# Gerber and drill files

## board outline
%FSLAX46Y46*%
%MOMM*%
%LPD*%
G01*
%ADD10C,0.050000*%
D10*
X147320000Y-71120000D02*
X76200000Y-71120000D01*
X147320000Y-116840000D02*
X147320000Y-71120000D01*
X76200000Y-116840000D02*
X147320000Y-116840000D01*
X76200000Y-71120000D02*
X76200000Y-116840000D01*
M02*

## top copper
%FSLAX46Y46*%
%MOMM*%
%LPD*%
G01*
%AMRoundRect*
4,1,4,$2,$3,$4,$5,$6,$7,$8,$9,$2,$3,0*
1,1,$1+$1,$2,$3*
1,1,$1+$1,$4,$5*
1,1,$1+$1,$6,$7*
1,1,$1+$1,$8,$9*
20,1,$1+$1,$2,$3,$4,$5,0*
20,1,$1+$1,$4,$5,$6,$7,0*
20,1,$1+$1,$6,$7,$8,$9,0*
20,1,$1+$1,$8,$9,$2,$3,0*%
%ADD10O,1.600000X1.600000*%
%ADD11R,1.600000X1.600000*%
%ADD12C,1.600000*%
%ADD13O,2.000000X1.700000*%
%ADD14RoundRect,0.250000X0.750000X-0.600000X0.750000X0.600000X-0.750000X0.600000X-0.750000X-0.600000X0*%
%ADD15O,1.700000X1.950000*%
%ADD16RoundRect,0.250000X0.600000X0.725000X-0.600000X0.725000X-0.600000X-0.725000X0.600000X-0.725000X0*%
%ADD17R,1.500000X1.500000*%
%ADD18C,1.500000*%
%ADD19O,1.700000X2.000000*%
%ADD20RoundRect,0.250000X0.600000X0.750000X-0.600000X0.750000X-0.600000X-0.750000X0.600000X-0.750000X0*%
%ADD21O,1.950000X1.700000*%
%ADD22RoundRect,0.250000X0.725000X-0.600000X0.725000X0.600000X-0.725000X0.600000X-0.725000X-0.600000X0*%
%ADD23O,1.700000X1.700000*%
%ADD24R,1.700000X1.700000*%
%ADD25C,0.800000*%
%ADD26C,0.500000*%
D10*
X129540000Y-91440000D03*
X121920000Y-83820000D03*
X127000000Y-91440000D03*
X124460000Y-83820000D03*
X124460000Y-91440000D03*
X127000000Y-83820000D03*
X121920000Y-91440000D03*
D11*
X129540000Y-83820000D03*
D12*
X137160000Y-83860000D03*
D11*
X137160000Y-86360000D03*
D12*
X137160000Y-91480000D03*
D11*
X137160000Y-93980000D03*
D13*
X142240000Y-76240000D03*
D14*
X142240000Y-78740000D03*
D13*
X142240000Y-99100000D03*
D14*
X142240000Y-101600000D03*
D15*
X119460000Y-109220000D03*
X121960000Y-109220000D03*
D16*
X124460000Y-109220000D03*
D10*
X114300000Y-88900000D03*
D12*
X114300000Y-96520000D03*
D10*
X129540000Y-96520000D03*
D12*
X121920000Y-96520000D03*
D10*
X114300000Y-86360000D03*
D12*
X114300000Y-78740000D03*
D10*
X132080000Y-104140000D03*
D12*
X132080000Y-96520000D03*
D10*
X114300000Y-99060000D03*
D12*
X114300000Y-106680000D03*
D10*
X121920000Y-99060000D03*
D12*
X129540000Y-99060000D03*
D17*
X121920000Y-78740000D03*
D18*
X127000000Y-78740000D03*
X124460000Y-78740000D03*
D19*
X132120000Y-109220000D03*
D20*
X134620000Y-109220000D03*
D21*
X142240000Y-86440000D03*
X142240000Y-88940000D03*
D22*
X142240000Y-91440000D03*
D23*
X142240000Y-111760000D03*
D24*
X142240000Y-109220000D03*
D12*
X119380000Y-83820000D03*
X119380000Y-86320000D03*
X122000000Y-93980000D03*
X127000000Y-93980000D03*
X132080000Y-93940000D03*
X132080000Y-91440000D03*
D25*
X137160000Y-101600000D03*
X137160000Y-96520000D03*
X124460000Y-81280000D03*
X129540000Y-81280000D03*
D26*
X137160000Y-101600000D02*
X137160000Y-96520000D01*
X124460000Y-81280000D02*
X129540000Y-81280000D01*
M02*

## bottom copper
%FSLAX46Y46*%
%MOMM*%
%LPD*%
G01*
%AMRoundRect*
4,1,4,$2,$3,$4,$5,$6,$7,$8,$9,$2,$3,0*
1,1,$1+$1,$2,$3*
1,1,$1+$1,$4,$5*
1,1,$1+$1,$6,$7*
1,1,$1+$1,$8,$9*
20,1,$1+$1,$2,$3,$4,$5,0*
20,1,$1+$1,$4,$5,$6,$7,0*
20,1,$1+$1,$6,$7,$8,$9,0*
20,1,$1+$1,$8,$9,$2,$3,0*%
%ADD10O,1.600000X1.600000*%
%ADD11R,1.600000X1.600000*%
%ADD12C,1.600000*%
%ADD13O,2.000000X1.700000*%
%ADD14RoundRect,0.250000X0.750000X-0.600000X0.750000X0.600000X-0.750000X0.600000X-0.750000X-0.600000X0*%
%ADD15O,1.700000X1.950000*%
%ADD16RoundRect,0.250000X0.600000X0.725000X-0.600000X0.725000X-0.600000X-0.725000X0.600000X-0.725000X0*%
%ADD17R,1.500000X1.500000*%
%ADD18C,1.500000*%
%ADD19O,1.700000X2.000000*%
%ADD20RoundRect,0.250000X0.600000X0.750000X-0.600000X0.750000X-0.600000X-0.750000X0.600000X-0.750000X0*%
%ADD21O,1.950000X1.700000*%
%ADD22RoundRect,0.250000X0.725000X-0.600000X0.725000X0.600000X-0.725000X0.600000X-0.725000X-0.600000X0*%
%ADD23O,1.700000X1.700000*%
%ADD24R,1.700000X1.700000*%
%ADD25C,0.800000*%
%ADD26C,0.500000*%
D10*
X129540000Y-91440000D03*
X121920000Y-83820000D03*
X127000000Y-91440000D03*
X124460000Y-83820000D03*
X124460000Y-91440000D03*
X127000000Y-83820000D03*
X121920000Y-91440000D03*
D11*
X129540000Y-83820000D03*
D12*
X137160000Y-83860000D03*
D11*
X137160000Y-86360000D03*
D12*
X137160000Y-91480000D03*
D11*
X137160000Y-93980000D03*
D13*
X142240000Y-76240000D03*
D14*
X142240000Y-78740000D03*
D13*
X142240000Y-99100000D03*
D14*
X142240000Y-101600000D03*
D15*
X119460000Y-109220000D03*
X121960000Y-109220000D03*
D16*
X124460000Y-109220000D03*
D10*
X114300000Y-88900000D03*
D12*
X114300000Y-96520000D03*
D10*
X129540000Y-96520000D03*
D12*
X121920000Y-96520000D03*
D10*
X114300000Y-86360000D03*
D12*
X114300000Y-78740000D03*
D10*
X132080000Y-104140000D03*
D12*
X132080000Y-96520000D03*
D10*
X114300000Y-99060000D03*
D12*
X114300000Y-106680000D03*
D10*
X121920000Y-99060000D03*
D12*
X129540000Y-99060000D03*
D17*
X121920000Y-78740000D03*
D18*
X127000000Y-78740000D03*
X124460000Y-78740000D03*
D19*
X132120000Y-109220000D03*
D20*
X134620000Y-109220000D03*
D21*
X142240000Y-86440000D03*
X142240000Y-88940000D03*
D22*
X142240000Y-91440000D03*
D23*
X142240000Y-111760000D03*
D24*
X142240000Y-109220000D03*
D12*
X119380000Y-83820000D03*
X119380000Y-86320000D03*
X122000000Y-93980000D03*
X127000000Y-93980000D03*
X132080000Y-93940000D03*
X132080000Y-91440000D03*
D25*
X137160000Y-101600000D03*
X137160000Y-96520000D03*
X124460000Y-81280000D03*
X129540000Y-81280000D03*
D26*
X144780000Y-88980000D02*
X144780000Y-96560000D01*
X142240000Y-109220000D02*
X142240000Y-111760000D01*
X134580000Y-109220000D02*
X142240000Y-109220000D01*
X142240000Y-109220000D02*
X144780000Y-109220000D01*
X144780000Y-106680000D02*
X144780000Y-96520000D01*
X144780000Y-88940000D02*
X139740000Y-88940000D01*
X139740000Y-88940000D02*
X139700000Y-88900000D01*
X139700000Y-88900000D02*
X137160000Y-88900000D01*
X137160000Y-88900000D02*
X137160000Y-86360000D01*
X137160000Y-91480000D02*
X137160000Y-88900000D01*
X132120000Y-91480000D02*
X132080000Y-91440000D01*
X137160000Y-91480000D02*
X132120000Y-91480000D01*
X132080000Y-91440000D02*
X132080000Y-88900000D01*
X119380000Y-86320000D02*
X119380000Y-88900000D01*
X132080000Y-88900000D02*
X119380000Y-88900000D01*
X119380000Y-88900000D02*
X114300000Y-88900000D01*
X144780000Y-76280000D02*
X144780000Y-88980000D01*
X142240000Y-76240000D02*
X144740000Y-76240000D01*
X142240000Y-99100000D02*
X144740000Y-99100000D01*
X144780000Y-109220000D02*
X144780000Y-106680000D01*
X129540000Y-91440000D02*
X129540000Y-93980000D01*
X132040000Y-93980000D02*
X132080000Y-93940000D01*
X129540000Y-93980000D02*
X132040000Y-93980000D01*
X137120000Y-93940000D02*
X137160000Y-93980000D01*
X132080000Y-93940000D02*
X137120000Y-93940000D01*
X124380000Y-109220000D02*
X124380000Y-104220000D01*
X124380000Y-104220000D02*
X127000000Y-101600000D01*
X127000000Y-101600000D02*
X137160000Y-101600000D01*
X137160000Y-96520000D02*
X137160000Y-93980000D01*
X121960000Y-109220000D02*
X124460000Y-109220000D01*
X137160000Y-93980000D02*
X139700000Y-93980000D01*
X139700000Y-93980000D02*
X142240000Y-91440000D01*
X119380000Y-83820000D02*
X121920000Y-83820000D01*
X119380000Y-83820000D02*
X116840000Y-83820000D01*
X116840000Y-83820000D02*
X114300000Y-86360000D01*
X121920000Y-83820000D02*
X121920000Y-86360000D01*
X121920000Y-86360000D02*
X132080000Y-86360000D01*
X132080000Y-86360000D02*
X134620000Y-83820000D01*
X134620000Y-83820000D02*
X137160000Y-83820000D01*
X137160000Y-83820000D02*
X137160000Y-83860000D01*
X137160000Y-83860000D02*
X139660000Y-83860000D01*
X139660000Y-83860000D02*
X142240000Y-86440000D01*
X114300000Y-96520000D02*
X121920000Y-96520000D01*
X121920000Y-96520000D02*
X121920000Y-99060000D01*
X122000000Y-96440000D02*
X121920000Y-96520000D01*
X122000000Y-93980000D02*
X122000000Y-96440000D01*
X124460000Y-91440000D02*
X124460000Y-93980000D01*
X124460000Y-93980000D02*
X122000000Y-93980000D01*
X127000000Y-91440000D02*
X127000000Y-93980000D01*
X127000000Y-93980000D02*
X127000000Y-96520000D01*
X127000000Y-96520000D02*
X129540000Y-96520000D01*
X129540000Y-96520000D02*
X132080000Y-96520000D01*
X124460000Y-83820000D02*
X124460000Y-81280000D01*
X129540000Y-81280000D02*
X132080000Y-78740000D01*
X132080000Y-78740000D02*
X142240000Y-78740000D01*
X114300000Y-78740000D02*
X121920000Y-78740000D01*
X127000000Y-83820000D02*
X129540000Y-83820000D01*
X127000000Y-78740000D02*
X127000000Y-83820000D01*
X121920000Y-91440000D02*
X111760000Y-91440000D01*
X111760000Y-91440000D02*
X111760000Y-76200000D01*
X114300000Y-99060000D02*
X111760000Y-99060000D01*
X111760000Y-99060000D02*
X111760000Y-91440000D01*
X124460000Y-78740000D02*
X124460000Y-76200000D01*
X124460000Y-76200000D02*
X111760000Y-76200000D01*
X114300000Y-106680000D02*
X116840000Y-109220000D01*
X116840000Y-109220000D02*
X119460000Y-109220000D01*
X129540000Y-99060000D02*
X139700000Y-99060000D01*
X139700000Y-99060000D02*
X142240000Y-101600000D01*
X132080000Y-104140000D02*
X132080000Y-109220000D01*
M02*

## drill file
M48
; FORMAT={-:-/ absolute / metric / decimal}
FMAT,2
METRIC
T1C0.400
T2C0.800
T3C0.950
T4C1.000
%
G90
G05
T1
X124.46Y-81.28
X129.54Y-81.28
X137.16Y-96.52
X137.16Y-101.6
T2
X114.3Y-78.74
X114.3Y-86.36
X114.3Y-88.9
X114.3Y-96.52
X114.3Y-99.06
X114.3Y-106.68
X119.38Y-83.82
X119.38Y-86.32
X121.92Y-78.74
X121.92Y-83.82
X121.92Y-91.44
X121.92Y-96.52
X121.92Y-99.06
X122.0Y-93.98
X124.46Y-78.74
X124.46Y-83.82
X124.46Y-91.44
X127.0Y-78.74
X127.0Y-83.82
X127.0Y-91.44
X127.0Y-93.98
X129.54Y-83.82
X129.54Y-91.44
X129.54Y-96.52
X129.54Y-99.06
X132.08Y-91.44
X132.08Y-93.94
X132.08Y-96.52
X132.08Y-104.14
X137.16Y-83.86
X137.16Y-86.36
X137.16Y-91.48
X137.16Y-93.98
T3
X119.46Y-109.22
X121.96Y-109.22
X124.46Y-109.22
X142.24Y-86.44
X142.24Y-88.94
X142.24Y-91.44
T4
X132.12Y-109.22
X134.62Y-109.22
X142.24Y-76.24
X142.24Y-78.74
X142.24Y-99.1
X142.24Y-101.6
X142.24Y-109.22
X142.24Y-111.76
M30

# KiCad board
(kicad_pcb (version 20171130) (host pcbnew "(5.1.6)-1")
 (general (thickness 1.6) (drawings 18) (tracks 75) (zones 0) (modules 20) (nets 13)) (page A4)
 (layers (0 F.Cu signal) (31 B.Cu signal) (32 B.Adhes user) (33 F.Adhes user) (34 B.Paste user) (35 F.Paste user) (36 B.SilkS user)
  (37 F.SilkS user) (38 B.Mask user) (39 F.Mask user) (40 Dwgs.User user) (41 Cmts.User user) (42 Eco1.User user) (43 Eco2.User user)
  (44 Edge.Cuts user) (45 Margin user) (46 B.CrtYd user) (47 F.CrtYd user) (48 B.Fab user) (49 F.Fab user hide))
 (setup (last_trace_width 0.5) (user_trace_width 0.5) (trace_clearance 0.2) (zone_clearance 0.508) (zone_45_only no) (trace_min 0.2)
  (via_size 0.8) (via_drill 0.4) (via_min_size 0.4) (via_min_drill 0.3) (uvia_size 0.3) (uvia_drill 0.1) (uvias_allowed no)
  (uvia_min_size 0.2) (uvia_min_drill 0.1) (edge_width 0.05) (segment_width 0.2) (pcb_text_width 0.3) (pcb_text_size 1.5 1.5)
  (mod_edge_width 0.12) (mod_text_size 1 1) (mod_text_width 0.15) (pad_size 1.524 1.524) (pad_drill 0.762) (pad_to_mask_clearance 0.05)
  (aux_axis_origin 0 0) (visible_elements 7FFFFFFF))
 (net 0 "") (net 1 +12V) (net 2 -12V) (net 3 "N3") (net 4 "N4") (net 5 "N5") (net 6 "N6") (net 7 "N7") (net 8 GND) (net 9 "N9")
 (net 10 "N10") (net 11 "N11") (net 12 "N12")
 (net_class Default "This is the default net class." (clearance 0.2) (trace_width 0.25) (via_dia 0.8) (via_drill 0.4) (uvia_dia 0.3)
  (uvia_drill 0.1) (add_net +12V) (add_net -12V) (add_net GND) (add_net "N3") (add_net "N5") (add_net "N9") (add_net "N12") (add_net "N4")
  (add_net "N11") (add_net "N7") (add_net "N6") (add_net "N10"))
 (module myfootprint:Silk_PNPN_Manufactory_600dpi (layer F.Cu) (at 86.36 78.74)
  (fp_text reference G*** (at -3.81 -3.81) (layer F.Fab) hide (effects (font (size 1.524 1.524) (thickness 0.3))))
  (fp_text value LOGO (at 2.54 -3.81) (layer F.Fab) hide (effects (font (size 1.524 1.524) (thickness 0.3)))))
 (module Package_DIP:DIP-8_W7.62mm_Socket (layer F.Cu) (at 129.54 83.82 270)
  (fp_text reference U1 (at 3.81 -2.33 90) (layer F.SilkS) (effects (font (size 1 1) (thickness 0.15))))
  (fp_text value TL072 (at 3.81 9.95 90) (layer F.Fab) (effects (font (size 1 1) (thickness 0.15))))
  (pad 8 thru_hole oval (at 7.62 0 270) (size 1.6 1.6) (drill 0.8) (layers *.Cu *.Mask) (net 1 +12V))
  (pad 4 thru_hole oval (at 0 7.62 270) (size 1.6 1.6) (drill 0.8) (layers *.Cu *.Mask) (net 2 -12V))
  (pad 7 thru_hole oval (at 7.62 2.54 270) (size 1.6 1.6) (drill 0.8) (layers *.Cu *.Mask) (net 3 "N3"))
  (pad 3 thru_hole oval (at 0 5.08 270) (size 1.6 1.6) (drill 0.8) (layers *.Cu *.Mask) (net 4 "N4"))
  (pad 6 thru_hole oval (at 7.62 5.08 270) (size 1.6 1.6) (drill 0.8) (layers *.Cu *.Mask) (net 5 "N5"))
  (pad 2 thru_hole oval (at 0 2.54 270) (size 1.6 1.6) (drill 0.8) (layers *.Cu *.Mask) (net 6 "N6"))
  (pad 5 thru_hole oval (at 7.62 7.62 270) (size 1.6 1.6) (drill 0.8) (layers *.Cu *.Mask) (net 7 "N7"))
  (pad 1 thru_hole rect (at 0 0 270) (size 1.6 1.6) (drill 0.8) (layers *.Cu *.Mask) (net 6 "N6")))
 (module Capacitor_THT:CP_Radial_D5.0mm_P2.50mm (layer F.Cu) (at 137.16 86.36 90)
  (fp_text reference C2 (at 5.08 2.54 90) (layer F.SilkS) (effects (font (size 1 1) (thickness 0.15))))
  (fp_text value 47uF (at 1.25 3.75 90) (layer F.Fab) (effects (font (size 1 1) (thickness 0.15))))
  (pad 2 thru_hole circle (at 2.5 0 90) (size 1.6 1.6) (drill 0.8) (layers *.Cu *.Mask) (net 2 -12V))
  (pad 1 thru_hole rect (at 0 0 90) (size 1.6 1.6) (drill 0.8) (layers *.Cu *.Mask) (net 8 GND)))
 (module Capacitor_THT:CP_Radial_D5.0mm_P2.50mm (layer F.Cu) (at 137.16 93.98 90)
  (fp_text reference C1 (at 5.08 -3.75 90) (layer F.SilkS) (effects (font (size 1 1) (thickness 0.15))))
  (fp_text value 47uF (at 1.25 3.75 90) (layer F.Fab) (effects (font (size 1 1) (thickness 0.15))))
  (pad 2 thru_hole circle (at 2.5 0 90) (size 1.6 1.6) (drill 0.8) (layers *.Cu *.Mask) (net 8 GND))
  (pad 1 thru_hole rect (at 0 0 90) (size 1.6 1.6) (drill 0.8) (layers *.Cu *.Mask) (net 1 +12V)))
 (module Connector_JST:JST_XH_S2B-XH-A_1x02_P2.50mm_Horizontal (layer F.Cu) (at 142.24 78.74 90)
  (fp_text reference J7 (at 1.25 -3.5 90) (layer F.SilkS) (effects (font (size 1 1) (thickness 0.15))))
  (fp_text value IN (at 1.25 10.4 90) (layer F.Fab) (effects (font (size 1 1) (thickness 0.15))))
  (pad 2 thru_hole oval (at 2.5 0 90) (size 1.7 2) (drill 1) (layers *.Cu *.Mask) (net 8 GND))
  (pad 1 thru_hole roundrect (at 0 0 90) (size 1.7 2) (drill 1) (layers *.Cu *.Mask) (roundrect_rratio 0.147059) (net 4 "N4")))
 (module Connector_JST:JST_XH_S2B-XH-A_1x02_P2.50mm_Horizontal (layer F.Cu) (at 142.24 101.6 90)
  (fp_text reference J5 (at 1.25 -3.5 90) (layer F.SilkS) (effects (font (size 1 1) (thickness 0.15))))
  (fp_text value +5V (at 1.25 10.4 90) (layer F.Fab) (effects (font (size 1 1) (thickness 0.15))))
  (pad 2 thru_hole oval (at 2.5 0 90) (size 1.7 2) (drill 1) (layers *.Cu *.Mask) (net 8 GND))
  (pad 1 thru_hole roundrect (at 0 0 90) (size 1.7 2) (drill 1) (layers *.Cu *.Mask) (roundrect_rratio 0.147059) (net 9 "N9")))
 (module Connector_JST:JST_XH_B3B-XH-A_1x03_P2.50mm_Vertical (layer F.Cu) (at 124.46 109.22 180)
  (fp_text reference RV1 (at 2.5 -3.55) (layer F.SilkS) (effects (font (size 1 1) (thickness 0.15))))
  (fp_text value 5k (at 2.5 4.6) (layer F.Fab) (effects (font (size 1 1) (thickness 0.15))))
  (pad 3 thru_hole oval (at 5 0 180) (size 1.7 1.95) (drill 0.95) (layers *.Cu *.Mask) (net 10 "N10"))
  (pad 2 thru_hole oval (at 2.5 0 180) (size 1.7 1.95) (drill 0.95) (layers *.Cu *.Mask) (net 1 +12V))
  (pad 1 thru_hole roundrect (at 0 0 180) (size 1.7 1.95) (drill 0.95) (layers *.Cu *.Mask) (roundrect_rratio 0.147059) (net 1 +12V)))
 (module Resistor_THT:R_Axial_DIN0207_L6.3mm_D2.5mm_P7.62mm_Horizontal (layer F.Cu) (at 114.3 96.52 90)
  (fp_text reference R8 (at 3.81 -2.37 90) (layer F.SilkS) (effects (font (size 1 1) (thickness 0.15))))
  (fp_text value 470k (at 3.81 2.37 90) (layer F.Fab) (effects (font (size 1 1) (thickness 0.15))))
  (pad 2 thru_hole oval (at 7.62 0 90) (size 1.6 1.6) (drill 0.8) (layers *.Cu *.Mask) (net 8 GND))
  (pad 1 thru_hole circle (at 0 0 90) (size 1.6 1.6) (drill 0.8) (layers *.Cu *.Mask) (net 5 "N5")))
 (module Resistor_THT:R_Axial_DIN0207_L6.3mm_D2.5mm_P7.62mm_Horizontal (layer F.Cu) (at 121.92 96.52)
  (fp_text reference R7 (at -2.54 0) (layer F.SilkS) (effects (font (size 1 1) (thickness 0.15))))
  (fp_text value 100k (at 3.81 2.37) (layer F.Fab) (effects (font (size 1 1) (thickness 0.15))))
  (pad 2 thru_hole oval (at 7.62 0) (size 1.6 1.6) (drill 0.8) (layers *.Cu *.Mask) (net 3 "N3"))
  (pad 1 thru_hole circle (at 0 0) (size 1.6 1.6) (drill 0.8) (layers *.Cu *.Mask) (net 5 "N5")))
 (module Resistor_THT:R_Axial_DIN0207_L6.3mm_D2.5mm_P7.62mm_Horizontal (layer F.Cu) (at 114.3 78.74 270)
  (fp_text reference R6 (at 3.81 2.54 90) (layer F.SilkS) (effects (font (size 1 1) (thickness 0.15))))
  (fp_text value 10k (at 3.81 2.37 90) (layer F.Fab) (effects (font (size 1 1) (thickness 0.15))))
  (pad 2 thru_hole oval (at 7.62 0 270) (size 1.6 1.6) (drill 0.8) (layers *.Cu *.Mask) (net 2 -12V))
  (pad 1 thru_hole circle (at 0 0 270) (size 1.6 1.6) (drill 0.8) (layers *.Cu *.Mask) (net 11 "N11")))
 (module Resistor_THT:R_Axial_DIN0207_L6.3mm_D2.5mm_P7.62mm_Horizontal (layer F.Cu) (at 132.08 96.52 270)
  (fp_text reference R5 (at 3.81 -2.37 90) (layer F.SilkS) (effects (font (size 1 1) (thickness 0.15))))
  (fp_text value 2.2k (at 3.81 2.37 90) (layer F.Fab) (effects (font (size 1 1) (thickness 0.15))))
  (pad 2 thru_hole oval (at 7.62 0 270) (size 1.6 1.6) (drill 0.8) (layers *.Cu *.Mask) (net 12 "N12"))
  (pad 1 thru_hole circle (at 0 0 270) (size 1.6 1.6) (drill 0.8) (layers *.Cu *.Mask) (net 3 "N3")))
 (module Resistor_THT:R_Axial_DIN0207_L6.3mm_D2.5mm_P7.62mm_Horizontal (layer F.Cu) (at 114.3 106.68 90)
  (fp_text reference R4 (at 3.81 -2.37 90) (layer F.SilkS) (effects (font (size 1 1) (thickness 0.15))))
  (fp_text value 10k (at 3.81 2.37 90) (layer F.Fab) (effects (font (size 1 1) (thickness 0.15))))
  (pad 2 thru_hole oval (at 7.62 0 90) (size 1.6 1.6) (drill 0.8) (layers *.Cu *.Mask) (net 7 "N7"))
  (pad 1 thru_hole circle (at 0 0 90) (size 1.6 1.6) (drill 0.8) (layers *.Cu *.Mask) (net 10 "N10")))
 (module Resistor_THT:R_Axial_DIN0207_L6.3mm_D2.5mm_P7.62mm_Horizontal (layer F.Cu) (at 129.54 99.06 180)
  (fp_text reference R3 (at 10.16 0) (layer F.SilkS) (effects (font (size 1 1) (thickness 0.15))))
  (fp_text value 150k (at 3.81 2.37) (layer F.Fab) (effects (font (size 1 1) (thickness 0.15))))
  (pad 2 thru_hole oval (at 7.62 0 180) (size 1.6 1.6) (drill 0.8) (layers *.Cu *.Mask) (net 5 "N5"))
  (pad 1 thru_hole circle (at 0 0 180) (size 1.6 1.6) (drill 0.8) (layers *.Cu *.Mask) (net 9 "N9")))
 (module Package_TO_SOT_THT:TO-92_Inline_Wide (layer F.Cu) (at 121.92 78.74)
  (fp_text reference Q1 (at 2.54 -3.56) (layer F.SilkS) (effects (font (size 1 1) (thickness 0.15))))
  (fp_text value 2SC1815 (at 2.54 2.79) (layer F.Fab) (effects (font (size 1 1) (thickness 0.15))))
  (pad 1 thru_hole rect (at 0 0 90) (size 1.5 1.5) (drill 0.8) (layers *.Cu *.Mask) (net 11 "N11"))
  (pad 3 thru_hole circle (at 5.08 0 90) (size 1.5 1.5) (drill 0.8) (layers *.Cu *.Mask) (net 6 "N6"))
  (pad 2 thru_hole circle (at 2.54 0 90) (size 1.5 1.5) (drill 0.8) (layers *.Cu *.Mask) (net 7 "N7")))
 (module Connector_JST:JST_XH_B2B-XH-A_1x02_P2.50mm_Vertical (layer F.Cu) (at 134.62 109.22 180)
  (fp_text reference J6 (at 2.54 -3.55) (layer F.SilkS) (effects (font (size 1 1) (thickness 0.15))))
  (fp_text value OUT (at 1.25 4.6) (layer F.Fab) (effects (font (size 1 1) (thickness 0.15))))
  (pad 2 thru_hole oval (at 2.5 0 180) (size 1.7 2) (drill 1) (layers *.Cu *.Mask) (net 12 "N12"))
  (pad 1 thru_hole roundrect (at 0 0 180) (size 1.7 2) (drill 1) (layers *.Cu *.Mask) (roundrect_rratio 0.147059) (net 8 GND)))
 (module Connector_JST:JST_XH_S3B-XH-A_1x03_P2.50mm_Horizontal (layer F.Cu) (at 142.24 91.44 90)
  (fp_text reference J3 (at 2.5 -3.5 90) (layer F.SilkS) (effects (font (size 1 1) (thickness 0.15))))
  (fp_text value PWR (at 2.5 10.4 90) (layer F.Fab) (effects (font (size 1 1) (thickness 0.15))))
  (pad 3 thru_hole oval (at 5 0 90) (size 1.7 1.95) (drill 0.95) (layers *.Cu *.Mask) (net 2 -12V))
  (pad 2 thru_hole oval (at 2.5 0 90) (size 1.7 1.95) (drill 0.95) (layers *.Cu *.Mask) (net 8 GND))
  (pad 1 thru_hole roundrect (at 0 0 90) (size 1.7 1.95) (drill 0.95) (layers *.Cu *.Mask) (roundrect_rratio 0.147059) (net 1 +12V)))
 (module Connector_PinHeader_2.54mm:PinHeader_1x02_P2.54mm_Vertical (layer F.Cu) (at 142.24 109.22)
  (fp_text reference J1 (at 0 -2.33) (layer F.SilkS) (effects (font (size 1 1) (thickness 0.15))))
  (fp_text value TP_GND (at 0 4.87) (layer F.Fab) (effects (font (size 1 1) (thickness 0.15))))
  (pad 2 thru_hole oval (at 0 2.54) (size 1.7 1.7) (drill 1) (layers *.Cu *.Mask) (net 8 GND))
  (pad 1 thru_hole rect (at 0 0) (size 1.7 1.7) (drill 1) (layers *.Cu *.Mask) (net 8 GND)))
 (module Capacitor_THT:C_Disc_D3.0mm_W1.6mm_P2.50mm (layer F.Cu) (at 119.38 86.32 90)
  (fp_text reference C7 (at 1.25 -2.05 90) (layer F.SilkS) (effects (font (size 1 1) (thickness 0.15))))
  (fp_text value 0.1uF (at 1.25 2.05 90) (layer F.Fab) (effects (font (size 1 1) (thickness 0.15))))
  (pad 2 thru_hole circle (at 2.5 0 90) (size 1.6 1.6) (drill 0.8) (layers *.Cu *.Mask) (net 2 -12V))
  (pad 1 thru_hole circle (at 0 0 90) (size 1.6 1.6) (drill 0.8) (layers *.Cu *.Mask) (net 8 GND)))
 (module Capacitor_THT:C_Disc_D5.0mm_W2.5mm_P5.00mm (layer F.Cu) (at 127 93.98 180)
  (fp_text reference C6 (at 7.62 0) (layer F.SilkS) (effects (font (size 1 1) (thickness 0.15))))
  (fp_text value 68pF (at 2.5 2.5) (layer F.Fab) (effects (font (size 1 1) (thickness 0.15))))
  (pad 2 thru_hole circle (at 5 0 180) (size 1.6 1.6) (drill 0.8) (layers *.Cu *.Mask) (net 5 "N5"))
  (pad 1 thru_hole circle (at 0 0 180) (size 1.6 1.6) (drill 0.8) (layers *.Cu *.Mask) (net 3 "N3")))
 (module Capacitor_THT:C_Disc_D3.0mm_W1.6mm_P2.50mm (layer F.Cu) (at 132.08 91.44 270)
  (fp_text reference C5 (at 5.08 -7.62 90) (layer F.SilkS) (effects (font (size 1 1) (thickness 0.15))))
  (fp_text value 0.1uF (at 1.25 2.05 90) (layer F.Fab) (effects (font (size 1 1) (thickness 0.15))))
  (pad 2 thru_hole circle (at 2.5 0 270) (size 1.6 1.6) (drill 0.8) (layers *.Cu *.Mask) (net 1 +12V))
  (pad 1 thru_hole circle (at 0 0 270) (size 1.6 1.6) (drill 0.8) (layers *.Cu *.Mask) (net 8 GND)))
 (gr_line (start 147.32 71.12) (end 76.2 71.12) (layer Edge.Cuts) (width 0.05))
 (gr_line (start 147.32 116.84) (end 147.32 71.12) (layer Edge.Cuts) (width 0.05))
 (gr_line (start 76.2 116.84) (end 147.32 116.84) (layer Edge.Cuts) (width 0.05))
 (gr_line (start 76.2 71.12) (end 76.2 116.84) (layer Edge.Cuts) (width 0.05))
 (segment (start 144.78 88.98) (end 144.78 96.56) (width 0.5) (layer B.Cu) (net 8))
 (segment (start 142.24 109.22) (end 142.24 111.76) (width 0.5) (layer B.Cu) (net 8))
 (segment (start 134.58 109.22) (end 142.24 109.22) (width 0.5) (layer B.Cu) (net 8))
 (segment (start 142.24 109.22) (end 144.78 109.22) (width 0.5) (layer B.Cu) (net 8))
 (segment (start 144.78 106.68) (end 144.78 96.52) (width 0.5) (layer B.Cu) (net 8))
 (segment (start 144.78 88.94) (end 139.74 88.94) (width 0.5) (layer B.Cu) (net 8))
 (segment (start 139.74 88.94) (end 139.7 88.9) (width 0.5) (layer B.Cu) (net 8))
 (segment (start 139.7 88.9) (end 137.16 88.9) (width 0.5) (layer B.Cu) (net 8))
 (segment (start 137.16 88.9) (end 137.16 86.36) (width 0.5) (layer B.Cu) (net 8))
 (segment (start 137.16 91.48) (end 137.16 88.9) (width 0.5) (layer B.Cu) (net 8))
 (segment (start 132.12 91.48) (end 132.08 91.44) (width 0.5) (layer B.Cu) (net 8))
 (segment (start 137.16 91.48) (end 132.12 91.48) (width 0.5) (layer B.Cu) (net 8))
 (segment (start 132.08 91.44) (end 132.08 88.9) (width 0.5) (layer B.Cu) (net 8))
 (segment (start 119.38 86.32) (end 119.38 88.9) (width 0.5) (layer B.Cu) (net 8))
 (segment (start 132.08 88.9) (end 119.38 88.9) (width 0.5) (layer B.Cu) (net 8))
 (segment (start 119.38 88.9) (end 114.3 88.9) (width 0.5) (layer B.Cu) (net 8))
 (segment (start 144.78 76.28) (end 144.78 88.98) (width 0.5) (layer B.Cu) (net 8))
 (segment (start 142.24 76.24) (end 144.74 76.24) (width 0.5) (layer B.Cu) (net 8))
 (segment (start 142.24 99.1) (end 144.74 99.1) (width 0.5) (layer B.Cu) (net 8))
 (segment (start 144.78 109.22) (end 144.78 106.68) (width 0.5) (layer B.Cu) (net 8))
 (segment (start 129.54 91.44) (end 129.54 93.98) (width 0.5) (layer B.Cu) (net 1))
 (segment (start 132.04 93.98) (end 132.08 93.94) (width 0.5) (layer B.Cu) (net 1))
 (segment (start 129.54 93.98) (end 132.04 93.98) (width 0.5) (layer B.Cu) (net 1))
 (segment (start 137.12 93.94) (end 137.16 93.98) (width 0.5) (layer B.Cu) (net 1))
 (segment (start 132.08 93.94) (end 137.12 93.94) (width 0.5) (layer B.Cu) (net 1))
 (segment (start 124.38 109.22) (end 124.38 104.22) (width 0.5) (layer B.Cu) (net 1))
 (segment (start 124.38 104.22) (end 127 101.6) (width 0.5) (layer B.Cu) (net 1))
 (segment (start 127 101.6) (end 137.16 101.6) (width 0.5) (layer B.Cu) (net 1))
 (via (at 137.16 101.6) (size 0.8) (drill 0.4) (layers F.Cu B.Cu) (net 1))
 (segment (start 137.16 101.6) (end 137.16 96.52) (width 0.5) (layer F.Cu) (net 1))
 (via (at 137.16 96.52) (size 0.8) (drill 0.4) (layers F.Cu B.Cu) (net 1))
 (segment (start 137.16 96.52) (end 137.16 93.98) (width 0.5) (layer B.Cu) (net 1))
 (segment (start 121.96 109.22) (end 124.46 109.22) (width 0.5) (layer B.Cu) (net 1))
 (segment (start 137.16 93.98) (end 139.7 93.98) (width 0.5) (layer B.Cu) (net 1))
 (segment (start 139.7 93.98) (end 142.24 91.44) (width 0.5) (layer B.Cu) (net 1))
 (segment (start 119.38 83.82) (end 121.92 83.82) (width 0.5) (layer B.Cu) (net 2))
 (segment (start 119.38 83.82) (end 116.84 83.82) (width 0.5) (layer B.Cu) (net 2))
 (segment (start 116.84 83.82) (end 114.3 86.36) (width 0.5) (layer B.Cu) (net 2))
 (segment (start 121.92 83.82) (end 121.92 86.36) (width 0.5) (layer B.Cu) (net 2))
 (segment (start 121.92 86.36) (end 132.08 86.36) (width 0.5) (layer B.Cu) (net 2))
 (segment (start 132.08 86.36) (end 134.62 83.82) (width 0.5) (layer B.Cu) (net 2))
 (segment (start 134.62 83.82) (end 137.16 83.82) (width 0.5) (layer B.Cu) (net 2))
 (segment (start 137.16 83.82) (end 137.16 83.86) (width 0.5) (layer B.Cu) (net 2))
 (segment (start 137.16 83.86) (end 139.66 83.86) (width 0.5) (layer B.Cu) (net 2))
 (segment (start 139.66 83.86) (end 142.24 86.44) (width 0.5) (layer B.Cu) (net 2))
 (segment (start 114.3 96.52) (end 121.92 96.52) (width 0.5) (layer B.Cu) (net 5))
 (segment (start 121.92 96.52) (end 121.92 99.06) (width 0.5) (layer B.Cu) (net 5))
 (segment (start 122 96.44) (end 121.92 96.52) (width 0.5) (layer B.Cu) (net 5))
 (segment (start 122 93.98) (end 122 96.44) (width 0.5) (layer B.Cu) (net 5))
 (segment (start 124.46 91.44) (end 124.46 93.98) (width 0.5) (layer B.Cu) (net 5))
 (segment (start 124.46 93.98) (end 122 93.98) (width 0.5) (layer B.Cu) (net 5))
 (segment (start 127 91.44) (end 127 93.98) (width 0.5) (layer B.Cu) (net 3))
 (segment (start 127 93.98) (end 127 96.52) (width 0.5) (layer B.Cu) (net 3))
 (segment (start 127 96.52) (end 129.54 96.52) (width 0.5) (layer B.Cu) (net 3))
 (segment (start 129.54 96.52) (end 132.08 96.52) (width 0.5) (layer B.Cu) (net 3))
 (segment (start 124.46 83.82) (end 124.46 81.28) (width 0.5) (layer B.Cu) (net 4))
 (via (at 124.46 81.28) (size 0.8) (drill 0.4) (layers F.Cu B.Cu) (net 4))
 (segment (start 124.46 81.28) (end 129.54 81.28) (width 0.5) (layer F.Cu) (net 4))
 (via (at 129.54 81.28) (size 0.8) (drill 0.4) (layers F.Cu B.Cu) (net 4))
 (segment (start 129.54 81.28) (end 132.08 78.74) (width 0.5) (layer B.Cu) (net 4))
 (segment (start 132.08 78.74) (end 142.24 78.74) (width 0.5) (layer B.Cu) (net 4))
 (segment (start 114.3 78.74) (end 121.92 78.74) (width 0.5) (layer B.Cu) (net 11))
 (segment (start 127 83.82) (end 129.54 83.82) (width 0.5) (layer B.Cu) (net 6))
 (segment (start 127 78.74) (end 127 83.82) (width 0.5) (layer B.Cu) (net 6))
 (segment (start 121.92 91.44) (end 111.76 91.44) (width 0.5) (layer B.Cu) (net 7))
 (segment (start 111.76 91.44) (end 111.76 76.2) (width 0.5) (layer B.Cu) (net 7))
 (segment (start 114.3 99.06) (end 111.76 99.06) (width 0.5) (layer B.Cu) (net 7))
 (segment (start 111.76 99.06) (end 111.76 91.44) (width 0.5) (layer B.Cu) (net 7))
 (segment (start 124.46 78.74) (end 124.46 76.2) (width 0.5) (layer B.Cu) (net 7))
 (segment (start 124.46 76.2) (end 111.76 76.2) (width 0.5) (layer B.Cu) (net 7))
 (segment (start 114.3 106.68) (end 116.84 109.22) (width 0.5) (layer B.Cu) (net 10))
 (segment (start 116.84 109.22) (end 119.46 109.22) (width 0.5) (layer B.Cu) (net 10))
 (segment (start 129.54 99.06) (end 139.7 99.06) (width 0.5) (layer B.Cu) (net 9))
 (segment (start 139.7 99.06) (end 142.24 101.6) (width 0.5) (layer B.Cu) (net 9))
 (segment (start 132.08 104.14) (end 132.08 109.22) (width 0.5) (layer B.Cu) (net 12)))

